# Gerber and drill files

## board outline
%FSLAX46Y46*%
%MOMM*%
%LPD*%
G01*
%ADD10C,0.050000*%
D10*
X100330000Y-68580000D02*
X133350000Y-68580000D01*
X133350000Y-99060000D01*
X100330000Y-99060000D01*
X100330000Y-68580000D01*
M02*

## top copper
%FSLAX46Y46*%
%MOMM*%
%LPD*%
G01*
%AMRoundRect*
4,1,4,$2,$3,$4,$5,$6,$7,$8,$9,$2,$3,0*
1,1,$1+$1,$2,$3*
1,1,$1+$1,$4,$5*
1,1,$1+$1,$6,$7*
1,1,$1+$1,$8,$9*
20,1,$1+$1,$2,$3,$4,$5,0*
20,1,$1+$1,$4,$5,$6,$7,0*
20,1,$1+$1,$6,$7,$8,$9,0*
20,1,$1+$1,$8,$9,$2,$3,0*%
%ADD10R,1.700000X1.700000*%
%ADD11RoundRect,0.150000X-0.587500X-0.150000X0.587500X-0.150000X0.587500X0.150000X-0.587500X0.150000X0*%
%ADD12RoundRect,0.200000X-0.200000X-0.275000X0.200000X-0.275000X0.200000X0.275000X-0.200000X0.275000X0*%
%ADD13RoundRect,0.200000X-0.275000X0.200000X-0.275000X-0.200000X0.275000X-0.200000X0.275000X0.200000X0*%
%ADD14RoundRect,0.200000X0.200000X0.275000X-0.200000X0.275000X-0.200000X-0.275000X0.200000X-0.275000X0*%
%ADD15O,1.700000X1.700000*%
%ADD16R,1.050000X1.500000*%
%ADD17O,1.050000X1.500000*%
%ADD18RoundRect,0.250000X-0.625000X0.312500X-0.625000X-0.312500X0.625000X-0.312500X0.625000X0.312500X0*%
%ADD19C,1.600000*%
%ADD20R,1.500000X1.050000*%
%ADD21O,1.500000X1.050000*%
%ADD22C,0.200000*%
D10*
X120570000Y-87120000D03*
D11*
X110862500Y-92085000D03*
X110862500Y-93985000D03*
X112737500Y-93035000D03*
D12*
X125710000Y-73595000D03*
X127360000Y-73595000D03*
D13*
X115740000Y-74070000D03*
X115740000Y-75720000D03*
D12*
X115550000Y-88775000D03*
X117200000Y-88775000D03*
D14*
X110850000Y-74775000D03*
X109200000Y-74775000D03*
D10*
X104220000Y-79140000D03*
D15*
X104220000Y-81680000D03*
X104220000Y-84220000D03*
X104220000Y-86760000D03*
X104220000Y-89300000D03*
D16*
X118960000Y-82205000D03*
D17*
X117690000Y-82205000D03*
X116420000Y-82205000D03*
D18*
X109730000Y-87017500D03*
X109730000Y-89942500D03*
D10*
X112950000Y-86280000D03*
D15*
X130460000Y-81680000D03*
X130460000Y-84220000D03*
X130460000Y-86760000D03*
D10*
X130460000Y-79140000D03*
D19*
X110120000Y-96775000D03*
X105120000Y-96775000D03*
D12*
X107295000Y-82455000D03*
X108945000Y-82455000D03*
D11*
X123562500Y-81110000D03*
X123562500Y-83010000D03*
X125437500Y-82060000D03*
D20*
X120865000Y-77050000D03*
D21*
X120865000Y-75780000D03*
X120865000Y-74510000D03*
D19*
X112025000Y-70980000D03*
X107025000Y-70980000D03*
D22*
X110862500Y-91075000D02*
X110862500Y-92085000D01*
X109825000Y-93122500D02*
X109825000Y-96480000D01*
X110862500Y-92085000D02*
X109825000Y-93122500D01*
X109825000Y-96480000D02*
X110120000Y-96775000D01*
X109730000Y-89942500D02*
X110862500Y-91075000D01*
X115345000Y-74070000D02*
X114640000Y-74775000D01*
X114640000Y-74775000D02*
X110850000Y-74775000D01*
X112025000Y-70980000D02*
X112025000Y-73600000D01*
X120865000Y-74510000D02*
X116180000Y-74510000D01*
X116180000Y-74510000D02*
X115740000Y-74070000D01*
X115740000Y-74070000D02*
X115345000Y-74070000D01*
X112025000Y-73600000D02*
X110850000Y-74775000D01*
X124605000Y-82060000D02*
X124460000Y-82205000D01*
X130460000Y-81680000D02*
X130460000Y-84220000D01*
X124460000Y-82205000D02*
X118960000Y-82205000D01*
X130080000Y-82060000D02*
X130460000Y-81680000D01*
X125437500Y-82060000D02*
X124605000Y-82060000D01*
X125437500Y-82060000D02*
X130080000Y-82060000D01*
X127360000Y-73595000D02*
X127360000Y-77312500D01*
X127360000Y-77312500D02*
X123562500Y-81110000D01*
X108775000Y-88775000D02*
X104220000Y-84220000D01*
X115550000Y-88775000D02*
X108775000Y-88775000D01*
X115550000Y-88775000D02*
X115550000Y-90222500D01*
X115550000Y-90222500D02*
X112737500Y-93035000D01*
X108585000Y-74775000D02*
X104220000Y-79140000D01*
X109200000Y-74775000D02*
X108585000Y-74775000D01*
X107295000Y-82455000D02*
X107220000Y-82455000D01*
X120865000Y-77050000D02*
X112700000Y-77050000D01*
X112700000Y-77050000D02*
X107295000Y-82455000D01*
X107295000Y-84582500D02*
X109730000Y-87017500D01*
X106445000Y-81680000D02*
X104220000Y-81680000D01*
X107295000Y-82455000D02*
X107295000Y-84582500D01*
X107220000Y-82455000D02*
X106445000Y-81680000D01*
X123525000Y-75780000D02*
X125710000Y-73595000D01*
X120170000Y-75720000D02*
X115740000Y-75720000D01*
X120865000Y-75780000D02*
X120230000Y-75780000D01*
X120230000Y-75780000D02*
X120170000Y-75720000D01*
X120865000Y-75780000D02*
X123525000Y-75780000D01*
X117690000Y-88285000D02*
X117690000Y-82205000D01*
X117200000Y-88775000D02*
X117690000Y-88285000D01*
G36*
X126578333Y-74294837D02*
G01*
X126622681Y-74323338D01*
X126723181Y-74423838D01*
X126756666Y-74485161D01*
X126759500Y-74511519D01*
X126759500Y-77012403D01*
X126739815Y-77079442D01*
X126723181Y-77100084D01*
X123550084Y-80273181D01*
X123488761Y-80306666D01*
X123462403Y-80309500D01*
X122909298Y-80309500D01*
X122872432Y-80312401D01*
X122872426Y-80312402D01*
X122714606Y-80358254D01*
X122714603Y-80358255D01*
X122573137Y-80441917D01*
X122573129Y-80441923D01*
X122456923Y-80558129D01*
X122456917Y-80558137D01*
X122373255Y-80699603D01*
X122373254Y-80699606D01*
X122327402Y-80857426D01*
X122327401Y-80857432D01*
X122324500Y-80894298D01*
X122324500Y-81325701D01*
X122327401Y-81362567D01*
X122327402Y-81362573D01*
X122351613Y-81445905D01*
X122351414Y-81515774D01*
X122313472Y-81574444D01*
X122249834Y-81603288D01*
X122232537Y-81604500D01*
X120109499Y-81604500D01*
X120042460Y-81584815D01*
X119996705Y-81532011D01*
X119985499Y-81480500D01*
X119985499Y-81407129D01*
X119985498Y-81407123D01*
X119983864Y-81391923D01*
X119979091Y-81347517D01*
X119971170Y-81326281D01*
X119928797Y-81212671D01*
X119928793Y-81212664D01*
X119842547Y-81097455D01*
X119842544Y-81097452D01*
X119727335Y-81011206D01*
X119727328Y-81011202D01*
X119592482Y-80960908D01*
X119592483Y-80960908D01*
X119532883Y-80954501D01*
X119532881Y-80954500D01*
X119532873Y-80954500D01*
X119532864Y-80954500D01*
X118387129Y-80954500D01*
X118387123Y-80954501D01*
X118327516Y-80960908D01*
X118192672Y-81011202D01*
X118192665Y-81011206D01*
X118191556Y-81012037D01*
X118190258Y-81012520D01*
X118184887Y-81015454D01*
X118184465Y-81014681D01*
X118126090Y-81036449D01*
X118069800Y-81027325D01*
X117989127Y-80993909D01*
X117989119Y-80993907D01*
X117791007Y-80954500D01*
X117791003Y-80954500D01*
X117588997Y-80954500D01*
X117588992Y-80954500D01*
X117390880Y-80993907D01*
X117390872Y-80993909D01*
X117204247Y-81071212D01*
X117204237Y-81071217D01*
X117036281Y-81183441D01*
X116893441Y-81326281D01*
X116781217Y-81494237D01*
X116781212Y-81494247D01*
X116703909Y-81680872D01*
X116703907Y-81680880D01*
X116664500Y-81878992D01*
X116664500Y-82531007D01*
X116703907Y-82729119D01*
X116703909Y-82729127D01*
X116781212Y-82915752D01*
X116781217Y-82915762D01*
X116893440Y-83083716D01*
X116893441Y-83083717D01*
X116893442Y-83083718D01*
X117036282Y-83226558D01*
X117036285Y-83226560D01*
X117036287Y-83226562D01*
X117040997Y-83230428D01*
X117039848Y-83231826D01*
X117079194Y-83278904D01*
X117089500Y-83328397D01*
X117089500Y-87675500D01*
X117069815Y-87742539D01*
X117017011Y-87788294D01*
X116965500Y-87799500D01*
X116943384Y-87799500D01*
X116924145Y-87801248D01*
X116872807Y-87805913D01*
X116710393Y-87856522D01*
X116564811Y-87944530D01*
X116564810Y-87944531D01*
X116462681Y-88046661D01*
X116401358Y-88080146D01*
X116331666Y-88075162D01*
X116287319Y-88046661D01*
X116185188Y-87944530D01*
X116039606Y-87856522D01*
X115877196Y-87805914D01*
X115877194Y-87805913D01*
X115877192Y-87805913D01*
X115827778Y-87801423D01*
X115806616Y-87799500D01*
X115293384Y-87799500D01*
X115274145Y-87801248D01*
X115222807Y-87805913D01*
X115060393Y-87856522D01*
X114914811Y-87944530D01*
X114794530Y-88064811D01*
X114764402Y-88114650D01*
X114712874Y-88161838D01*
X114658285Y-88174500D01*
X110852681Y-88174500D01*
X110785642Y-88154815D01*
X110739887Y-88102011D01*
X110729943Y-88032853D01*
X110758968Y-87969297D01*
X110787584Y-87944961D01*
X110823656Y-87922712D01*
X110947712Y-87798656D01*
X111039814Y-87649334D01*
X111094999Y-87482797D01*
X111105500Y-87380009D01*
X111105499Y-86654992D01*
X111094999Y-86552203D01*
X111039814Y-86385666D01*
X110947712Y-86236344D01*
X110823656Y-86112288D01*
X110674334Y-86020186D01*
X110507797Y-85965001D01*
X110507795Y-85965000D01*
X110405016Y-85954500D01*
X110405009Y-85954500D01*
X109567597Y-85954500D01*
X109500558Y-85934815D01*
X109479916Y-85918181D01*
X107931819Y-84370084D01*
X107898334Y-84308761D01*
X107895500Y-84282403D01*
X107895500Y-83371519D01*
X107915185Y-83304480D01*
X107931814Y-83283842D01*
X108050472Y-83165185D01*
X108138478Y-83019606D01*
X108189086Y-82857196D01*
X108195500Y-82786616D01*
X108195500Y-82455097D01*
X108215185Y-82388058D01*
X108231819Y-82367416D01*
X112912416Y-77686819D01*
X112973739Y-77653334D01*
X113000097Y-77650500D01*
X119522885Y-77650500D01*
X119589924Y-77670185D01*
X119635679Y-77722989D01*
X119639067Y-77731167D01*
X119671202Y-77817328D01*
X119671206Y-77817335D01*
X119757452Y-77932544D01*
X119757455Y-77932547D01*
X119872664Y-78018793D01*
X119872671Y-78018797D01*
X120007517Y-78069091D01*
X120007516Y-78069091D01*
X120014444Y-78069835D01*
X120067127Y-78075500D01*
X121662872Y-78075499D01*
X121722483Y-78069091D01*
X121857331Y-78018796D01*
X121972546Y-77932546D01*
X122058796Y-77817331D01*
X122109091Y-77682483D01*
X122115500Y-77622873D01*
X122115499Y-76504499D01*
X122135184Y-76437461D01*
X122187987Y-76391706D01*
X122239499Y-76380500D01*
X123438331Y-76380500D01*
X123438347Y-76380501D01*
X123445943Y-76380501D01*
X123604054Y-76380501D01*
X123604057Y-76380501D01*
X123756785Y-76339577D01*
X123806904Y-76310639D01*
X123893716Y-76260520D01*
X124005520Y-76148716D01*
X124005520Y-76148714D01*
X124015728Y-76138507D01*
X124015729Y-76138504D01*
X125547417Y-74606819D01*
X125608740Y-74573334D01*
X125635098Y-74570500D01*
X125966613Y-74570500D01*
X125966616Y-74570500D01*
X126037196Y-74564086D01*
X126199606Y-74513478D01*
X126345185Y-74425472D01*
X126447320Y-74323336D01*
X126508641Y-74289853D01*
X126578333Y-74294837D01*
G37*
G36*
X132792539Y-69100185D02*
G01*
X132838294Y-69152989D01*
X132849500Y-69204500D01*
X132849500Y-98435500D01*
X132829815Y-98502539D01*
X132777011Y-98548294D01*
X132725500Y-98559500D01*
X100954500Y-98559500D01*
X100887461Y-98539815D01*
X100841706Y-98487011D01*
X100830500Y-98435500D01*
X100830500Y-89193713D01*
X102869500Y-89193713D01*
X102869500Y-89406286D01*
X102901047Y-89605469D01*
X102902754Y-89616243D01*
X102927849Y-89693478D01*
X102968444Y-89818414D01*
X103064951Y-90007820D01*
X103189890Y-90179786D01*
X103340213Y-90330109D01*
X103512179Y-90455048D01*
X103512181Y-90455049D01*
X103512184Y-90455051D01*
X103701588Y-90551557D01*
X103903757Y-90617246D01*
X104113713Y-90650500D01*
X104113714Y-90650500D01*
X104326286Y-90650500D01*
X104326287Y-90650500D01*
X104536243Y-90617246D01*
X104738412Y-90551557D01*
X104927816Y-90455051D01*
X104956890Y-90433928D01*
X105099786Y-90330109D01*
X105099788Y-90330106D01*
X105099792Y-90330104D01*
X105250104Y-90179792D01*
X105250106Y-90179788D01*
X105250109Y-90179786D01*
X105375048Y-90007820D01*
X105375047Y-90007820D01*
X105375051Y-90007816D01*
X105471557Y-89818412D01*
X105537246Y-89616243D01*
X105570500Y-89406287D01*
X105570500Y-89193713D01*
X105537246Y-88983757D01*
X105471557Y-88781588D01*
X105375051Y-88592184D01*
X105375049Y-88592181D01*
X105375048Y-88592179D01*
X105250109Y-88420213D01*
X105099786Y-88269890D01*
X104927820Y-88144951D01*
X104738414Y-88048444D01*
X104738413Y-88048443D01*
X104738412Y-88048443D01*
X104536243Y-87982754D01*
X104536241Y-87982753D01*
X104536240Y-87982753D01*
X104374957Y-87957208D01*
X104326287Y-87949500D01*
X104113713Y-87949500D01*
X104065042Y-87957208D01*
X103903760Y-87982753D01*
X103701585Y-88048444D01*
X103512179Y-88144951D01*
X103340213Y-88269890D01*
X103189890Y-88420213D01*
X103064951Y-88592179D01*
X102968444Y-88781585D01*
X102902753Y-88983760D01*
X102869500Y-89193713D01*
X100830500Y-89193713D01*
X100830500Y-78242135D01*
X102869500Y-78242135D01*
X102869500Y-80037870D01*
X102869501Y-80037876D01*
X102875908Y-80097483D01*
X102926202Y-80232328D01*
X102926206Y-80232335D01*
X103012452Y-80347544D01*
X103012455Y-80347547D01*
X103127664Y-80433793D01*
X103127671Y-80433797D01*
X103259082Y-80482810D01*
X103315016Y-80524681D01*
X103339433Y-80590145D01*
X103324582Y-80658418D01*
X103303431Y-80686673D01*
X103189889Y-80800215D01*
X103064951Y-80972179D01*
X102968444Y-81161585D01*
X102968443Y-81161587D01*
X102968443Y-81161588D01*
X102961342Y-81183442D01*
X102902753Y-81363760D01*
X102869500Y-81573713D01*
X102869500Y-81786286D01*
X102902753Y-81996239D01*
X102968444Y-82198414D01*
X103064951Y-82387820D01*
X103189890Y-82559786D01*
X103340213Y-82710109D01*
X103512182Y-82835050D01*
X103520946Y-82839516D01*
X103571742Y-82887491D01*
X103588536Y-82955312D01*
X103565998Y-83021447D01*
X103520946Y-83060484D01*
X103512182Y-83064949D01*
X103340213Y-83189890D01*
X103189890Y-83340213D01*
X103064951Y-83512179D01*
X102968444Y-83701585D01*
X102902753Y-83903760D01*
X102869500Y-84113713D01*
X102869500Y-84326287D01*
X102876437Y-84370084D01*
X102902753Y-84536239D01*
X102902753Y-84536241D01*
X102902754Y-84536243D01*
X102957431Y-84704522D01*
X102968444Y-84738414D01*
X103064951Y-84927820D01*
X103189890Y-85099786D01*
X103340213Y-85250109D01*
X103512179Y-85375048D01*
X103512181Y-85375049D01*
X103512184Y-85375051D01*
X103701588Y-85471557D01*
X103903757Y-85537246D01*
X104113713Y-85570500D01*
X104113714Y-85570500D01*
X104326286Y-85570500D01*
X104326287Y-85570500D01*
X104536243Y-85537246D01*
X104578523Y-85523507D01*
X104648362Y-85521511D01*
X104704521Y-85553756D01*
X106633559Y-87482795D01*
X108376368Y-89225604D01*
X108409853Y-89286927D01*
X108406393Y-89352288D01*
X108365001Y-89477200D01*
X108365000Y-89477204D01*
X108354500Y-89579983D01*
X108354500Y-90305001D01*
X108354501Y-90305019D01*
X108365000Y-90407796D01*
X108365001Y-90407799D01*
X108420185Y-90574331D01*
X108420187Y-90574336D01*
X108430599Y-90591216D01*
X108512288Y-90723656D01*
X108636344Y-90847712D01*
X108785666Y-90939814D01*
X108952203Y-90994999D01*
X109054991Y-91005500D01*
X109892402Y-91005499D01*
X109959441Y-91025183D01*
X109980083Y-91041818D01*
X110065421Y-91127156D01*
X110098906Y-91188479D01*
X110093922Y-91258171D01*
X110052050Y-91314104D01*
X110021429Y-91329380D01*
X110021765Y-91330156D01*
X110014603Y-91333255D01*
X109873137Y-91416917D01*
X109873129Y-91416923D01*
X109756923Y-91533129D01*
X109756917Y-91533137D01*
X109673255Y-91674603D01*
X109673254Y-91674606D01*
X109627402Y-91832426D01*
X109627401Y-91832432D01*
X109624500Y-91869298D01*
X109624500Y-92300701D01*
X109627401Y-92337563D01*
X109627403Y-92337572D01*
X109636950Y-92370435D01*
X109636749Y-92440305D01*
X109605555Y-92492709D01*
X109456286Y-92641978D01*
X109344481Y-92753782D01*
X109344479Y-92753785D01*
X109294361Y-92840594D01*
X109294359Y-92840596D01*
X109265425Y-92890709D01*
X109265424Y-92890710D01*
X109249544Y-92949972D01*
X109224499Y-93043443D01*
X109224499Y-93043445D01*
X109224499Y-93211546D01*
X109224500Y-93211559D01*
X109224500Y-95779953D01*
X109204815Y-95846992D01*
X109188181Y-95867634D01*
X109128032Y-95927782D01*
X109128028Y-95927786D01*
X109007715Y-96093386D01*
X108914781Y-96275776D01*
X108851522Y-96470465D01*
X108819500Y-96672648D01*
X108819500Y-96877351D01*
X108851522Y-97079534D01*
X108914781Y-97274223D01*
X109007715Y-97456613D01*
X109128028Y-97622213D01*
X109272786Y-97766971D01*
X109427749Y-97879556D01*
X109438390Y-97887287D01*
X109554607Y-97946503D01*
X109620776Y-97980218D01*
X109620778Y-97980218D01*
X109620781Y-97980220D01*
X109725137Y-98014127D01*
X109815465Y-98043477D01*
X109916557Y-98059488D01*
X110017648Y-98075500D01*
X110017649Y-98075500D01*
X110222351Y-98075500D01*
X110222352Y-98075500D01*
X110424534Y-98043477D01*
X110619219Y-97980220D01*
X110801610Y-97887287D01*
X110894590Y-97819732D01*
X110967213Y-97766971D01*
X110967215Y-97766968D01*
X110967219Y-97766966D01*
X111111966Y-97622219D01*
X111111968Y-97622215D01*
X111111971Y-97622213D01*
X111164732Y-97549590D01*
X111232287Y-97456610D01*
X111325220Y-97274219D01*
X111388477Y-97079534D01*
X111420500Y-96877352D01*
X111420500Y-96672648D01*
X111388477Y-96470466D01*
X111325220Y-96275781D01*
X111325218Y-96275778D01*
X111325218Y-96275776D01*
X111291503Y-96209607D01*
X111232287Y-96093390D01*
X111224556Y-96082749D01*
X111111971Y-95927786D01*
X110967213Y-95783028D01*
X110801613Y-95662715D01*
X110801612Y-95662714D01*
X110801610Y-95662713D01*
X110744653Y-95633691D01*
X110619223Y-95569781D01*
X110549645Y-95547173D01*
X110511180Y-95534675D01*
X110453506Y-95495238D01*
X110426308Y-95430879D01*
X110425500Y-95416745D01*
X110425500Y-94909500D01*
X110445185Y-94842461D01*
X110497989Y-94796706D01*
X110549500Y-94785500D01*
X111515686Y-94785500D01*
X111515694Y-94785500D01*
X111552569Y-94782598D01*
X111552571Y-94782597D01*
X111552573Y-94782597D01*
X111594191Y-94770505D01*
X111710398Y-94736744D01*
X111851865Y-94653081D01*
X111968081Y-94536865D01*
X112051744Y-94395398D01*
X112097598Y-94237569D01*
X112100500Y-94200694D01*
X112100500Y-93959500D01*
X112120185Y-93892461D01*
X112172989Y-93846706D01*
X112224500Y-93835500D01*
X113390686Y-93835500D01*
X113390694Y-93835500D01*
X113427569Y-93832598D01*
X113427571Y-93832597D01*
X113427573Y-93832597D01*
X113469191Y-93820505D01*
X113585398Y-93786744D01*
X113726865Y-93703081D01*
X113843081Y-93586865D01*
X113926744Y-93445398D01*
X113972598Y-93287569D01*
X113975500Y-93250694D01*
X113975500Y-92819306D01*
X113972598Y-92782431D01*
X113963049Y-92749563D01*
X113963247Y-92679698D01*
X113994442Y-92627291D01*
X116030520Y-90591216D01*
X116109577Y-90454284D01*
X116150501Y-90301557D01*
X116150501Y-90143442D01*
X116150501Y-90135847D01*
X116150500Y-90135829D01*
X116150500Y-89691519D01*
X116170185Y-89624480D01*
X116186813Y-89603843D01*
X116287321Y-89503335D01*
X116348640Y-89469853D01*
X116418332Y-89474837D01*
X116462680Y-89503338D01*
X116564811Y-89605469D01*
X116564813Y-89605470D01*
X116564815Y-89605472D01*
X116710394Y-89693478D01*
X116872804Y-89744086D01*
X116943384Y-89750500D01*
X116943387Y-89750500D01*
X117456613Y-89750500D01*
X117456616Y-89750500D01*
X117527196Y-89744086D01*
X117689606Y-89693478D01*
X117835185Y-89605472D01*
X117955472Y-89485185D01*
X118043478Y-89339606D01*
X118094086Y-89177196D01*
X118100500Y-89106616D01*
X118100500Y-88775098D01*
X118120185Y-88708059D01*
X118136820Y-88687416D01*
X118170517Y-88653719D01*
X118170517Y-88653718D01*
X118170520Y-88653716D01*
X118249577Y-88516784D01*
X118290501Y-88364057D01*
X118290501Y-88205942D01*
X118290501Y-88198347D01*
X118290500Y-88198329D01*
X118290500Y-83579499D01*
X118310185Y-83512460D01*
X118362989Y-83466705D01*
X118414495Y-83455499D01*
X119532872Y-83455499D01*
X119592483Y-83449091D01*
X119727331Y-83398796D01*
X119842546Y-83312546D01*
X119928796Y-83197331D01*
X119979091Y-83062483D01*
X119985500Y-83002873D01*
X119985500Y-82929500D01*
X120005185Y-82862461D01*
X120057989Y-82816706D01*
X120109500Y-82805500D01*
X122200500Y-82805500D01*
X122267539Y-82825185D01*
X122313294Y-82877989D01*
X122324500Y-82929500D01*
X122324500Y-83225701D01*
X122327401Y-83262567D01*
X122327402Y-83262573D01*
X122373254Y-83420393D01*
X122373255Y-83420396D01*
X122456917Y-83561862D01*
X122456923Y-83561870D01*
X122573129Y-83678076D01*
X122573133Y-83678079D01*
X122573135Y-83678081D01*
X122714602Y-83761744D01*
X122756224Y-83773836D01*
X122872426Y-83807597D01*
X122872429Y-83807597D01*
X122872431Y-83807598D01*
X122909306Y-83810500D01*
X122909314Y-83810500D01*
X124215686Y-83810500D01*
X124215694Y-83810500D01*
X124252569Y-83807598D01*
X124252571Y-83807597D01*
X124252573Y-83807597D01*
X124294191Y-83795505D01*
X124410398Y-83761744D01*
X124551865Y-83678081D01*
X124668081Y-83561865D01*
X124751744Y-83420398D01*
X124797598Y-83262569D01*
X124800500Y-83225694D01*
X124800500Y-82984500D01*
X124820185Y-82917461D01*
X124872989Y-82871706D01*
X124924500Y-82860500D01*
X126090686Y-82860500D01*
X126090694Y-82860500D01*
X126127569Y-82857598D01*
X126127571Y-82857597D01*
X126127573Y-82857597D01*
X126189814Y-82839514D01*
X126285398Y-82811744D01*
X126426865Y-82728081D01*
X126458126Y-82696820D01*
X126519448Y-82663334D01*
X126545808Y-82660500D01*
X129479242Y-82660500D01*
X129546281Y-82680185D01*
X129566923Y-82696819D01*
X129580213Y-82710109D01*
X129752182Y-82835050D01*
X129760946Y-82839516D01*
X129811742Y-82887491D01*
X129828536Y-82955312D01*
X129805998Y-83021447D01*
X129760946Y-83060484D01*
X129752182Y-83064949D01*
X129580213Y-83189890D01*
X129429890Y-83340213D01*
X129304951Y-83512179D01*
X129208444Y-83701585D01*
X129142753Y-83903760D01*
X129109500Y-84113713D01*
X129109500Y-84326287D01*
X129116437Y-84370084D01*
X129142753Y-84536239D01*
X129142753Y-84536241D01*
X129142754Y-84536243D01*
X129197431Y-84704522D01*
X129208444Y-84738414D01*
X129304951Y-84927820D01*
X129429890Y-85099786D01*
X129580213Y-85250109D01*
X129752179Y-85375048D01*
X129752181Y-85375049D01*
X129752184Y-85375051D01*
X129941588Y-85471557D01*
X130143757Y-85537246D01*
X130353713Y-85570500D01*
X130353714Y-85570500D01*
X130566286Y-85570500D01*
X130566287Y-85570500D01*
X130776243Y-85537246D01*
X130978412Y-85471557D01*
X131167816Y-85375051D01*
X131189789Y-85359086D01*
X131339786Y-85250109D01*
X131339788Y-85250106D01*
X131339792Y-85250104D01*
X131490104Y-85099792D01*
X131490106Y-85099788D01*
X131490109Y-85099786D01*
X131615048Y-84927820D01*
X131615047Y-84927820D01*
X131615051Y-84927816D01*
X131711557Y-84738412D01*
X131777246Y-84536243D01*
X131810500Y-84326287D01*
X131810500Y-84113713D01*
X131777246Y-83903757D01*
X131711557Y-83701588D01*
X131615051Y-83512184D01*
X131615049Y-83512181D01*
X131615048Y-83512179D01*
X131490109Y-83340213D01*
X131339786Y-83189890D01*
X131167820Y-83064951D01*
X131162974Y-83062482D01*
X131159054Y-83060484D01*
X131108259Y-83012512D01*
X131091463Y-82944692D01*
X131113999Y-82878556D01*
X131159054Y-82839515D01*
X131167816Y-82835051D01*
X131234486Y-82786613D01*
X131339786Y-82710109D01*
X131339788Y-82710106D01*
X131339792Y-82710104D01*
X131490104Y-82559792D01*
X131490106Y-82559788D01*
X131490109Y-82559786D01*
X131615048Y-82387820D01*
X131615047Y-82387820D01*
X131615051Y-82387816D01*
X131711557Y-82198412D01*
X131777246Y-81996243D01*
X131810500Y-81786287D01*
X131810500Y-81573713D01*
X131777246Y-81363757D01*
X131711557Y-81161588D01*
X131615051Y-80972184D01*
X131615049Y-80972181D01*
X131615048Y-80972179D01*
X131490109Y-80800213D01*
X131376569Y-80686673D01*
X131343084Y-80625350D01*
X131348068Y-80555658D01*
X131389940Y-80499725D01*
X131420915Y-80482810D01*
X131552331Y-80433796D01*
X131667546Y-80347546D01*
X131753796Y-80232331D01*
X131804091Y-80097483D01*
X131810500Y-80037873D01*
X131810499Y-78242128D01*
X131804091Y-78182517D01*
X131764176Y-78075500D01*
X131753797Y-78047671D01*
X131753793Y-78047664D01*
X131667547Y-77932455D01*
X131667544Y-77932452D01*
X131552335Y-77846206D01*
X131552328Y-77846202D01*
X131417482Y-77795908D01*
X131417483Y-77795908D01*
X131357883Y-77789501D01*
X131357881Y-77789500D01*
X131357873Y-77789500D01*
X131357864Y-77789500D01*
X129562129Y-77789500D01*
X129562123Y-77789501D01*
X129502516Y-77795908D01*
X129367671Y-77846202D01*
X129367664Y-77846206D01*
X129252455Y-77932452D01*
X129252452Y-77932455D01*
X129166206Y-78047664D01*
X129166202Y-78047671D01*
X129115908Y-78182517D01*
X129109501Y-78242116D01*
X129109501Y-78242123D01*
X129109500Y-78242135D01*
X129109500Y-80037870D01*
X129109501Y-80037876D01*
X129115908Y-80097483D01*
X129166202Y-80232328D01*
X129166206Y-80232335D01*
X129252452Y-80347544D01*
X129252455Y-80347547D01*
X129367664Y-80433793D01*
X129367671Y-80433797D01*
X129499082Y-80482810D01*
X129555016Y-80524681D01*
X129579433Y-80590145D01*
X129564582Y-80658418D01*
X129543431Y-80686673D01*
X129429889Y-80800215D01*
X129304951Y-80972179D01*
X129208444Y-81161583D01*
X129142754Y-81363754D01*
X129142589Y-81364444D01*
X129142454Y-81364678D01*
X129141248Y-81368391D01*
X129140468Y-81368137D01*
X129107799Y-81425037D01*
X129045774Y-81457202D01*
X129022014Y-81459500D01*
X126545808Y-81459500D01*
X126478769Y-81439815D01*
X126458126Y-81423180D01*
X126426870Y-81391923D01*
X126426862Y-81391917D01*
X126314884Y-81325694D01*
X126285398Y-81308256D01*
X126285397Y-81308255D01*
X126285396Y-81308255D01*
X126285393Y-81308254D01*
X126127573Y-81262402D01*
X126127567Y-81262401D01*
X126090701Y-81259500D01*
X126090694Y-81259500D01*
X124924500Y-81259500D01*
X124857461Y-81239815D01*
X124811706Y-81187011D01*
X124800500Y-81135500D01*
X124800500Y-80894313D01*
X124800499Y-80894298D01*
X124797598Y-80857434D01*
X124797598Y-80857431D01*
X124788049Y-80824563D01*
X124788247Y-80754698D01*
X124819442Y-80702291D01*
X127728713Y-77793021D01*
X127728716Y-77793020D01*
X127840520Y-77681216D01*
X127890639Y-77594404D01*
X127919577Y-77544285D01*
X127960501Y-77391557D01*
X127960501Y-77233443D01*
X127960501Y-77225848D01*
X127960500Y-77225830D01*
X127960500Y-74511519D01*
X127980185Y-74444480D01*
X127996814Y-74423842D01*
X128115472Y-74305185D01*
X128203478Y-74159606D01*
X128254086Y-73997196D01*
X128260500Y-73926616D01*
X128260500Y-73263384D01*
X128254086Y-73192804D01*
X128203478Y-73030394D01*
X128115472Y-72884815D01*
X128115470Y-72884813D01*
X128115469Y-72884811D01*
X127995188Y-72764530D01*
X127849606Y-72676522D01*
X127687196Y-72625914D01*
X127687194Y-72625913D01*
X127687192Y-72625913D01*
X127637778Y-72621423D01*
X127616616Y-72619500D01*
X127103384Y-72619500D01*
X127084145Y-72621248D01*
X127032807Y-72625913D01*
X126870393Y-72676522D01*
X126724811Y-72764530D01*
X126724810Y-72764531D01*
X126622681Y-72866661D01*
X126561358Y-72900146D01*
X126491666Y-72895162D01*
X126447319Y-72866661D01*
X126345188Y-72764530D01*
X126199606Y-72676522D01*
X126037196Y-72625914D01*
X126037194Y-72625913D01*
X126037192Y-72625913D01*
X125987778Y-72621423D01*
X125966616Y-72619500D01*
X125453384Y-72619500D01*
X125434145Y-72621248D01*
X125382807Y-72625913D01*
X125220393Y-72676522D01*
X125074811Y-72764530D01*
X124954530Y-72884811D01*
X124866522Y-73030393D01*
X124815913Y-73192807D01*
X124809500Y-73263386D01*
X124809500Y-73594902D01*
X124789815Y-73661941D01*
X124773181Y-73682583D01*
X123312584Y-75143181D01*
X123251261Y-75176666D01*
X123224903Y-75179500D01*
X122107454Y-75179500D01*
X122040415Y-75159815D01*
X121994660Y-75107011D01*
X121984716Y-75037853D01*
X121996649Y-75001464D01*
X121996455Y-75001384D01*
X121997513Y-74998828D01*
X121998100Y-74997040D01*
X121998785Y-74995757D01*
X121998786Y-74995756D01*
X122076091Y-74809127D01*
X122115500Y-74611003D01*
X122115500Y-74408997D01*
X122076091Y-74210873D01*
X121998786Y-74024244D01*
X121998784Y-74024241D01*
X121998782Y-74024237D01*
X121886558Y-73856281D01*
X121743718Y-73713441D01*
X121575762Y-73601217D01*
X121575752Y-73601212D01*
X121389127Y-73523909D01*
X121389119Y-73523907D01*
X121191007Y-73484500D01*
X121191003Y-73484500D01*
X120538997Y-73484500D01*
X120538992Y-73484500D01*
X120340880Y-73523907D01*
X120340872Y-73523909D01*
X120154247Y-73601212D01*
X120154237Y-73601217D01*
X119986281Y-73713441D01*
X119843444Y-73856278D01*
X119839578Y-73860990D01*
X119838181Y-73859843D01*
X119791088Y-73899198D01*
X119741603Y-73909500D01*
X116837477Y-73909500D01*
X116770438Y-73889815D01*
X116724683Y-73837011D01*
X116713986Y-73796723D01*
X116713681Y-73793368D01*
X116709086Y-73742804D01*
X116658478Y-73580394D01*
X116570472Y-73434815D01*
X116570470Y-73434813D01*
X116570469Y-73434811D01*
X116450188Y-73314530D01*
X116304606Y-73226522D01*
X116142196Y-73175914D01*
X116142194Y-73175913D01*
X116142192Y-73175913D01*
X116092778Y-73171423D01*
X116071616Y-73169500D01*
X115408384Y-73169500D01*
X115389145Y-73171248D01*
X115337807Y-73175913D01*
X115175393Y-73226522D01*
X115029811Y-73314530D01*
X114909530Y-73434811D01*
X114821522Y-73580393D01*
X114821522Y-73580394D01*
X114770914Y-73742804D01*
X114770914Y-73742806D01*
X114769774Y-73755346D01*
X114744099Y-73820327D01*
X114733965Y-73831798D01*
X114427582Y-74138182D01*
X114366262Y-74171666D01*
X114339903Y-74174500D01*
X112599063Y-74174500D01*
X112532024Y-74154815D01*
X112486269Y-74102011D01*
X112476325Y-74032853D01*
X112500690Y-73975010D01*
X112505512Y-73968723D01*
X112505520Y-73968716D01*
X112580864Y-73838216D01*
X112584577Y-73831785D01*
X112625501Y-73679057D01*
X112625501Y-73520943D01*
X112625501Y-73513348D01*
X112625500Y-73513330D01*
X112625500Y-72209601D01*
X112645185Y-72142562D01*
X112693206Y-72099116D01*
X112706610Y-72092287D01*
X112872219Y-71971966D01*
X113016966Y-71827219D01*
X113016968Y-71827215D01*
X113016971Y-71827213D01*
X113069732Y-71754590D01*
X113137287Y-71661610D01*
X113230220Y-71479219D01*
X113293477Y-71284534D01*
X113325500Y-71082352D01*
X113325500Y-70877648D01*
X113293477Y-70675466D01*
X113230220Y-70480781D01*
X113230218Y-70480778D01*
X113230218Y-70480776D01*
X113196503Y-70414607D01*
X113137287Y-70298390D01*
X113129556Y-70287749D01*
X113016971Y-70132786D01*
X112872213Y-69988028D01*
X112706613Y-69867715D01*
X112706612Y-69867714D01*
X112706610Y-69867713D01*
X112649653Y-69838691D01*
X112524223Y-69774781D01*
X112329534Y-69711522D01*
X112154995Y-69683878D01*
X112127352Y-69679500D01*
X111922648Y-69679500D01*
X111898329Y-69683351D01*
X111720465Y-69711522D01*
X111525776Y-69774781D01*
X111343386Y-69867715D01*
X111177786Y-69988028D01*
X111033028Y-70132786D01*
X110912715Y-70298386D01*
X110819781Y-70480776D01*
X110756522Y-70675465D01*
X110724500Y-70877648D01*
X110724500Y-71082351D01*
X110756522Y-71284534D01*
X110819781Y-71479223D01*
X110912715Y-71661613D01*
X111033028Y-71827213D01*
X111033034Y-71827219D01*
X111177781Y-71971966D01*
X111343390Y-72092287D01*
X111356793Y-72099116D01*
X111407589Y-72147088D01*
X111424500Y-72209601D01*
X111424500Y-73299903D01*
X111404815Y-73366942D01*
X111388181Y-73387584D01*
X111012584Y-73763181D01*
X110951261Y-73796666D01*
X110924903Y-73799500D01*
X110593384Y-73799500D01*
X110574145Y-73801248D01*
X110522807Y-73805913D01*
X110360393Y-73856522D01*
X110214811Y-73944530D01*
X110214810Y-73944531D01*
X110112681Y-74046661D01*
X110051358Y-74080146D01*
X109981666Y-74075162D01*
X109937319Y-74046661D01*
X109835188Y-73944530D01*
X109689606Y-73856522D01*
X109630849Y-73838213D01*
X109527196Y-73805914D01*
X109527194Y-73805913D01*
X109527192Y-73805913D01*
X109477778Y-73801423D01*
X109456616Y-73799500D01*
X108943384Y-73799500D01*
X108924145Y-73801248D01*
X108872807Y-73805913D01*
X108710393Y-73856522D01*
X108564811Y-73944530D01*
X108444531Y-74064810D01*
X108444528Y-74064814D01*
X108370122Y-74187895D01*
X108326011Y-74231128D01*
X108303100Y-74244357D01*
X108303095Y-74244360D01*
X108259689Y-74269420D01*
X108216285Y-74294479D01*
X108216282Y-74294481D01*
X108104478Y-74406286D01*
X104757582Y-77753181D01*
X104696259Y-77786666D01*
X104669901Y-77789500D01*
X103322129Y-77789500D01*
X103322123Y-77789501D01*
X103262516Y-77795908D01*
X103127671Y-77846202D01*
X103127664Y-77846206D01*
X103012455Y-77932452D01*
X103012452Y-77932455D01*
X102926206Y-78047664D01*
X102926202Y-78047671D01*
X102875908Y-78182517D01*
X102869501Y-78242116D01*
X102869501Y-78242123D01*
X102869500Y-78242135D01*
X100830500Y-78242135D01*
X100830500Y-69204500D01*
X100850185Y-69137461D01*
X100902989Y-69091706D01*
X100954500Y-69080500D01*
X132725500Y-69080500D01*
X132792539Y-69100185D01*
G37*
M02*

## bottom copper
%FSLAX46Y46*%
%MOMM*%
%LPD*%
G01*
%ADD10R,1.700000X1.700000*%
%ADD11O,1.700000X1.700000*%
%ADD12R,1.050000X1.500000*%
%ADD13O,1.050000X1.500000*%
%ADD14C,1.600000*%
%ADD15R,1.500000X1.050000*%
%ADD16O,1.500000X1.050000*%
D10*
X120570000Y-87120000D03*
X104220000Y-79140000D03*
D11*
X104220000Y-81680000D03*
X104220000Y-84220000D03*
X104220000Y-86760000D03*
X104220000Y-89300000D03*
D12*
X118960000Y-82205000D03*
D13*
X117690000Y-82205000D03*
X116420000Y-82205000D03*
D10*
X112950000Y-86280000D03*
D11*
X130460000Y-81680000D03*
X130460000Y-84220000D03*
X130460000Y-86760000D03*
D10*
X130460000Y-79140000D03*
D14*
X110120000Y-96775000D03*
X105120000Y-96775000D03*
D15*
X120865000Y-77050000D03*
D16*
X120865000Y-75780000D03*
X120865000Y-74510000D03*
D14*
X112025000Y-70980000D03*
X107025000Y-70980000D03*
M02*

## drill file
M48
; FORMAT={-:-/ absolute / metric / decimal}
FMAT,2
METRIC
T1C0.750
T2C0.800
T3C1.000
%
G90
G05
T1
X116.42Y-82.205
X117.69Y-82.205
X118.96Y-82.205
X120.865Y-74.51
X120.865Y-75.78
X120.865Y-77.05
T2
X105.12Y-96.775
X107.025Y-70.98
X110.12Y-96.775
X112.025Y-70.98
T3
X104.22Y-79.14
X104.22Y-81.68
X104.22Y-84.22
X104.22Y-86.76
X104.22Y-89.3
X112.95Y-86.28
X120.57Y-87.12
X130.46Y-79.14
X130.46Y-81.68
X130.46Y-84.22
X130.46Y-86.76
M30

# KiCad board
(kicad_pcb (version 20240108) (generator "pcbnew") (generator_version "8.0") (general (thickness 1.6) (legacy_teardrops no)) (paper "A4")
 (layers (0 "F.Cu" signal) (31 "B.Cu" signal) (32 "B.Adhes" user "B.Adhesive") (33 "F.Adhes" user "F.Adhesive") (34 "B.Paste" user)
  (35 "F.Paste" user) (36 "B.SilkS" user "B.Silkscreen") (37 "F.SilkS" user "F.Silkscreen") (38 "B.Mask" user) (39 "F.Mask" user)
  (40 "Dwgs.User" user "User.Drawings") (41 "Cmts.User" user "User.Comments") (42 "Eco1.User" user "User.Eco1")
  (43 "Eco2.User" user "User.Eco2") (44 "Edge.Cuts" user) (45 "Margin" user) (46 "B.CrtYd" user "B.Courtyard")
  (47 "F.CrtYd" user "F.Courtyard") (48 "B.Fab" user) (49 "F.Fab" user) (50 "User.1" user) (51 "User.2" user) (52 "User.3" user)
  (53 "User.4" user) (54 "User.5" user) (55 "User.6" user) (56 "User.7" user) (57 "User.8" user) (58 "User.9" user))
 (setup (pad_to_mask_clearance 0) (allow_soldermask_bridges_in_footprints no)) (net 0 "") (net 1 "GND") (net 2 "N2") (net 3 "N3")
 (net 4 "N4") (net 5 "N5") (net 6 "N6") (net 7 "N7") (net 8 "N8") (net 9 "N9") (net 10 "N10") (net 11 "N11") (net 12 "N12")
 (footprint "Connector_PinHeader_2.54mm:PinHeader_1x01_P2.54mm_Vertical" (layer "F.Cu") (at 120.57 87.12)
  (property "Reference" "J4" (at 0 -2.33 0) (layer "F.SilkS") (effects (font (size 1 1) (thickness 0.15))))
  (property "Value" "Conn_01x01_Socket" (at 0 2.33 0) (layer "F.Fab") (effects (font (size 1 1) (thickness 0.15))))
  (pad "1" thru_hole rect (at 0 0) (size 1.7 1.7) (drill 1) (layers "*.Cu" "*.Mask") (remove_unused_layers no) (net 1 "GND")))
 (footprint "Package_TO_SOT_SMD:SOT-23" (layer "F.Cu") (at 111.8 93.035)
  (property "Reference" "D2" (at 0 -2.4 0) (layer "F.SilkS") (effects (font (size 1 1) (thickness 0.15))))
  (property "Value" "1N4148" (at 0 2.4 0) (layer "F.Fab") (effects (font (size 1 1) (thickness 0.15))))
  (pad "1" smd roundrect (at -0.9375 -0.95) (size 1.475 0.6) (layers "F.Cu" "F.Paste" "F.Mask") (roundrect_rratio 0.25) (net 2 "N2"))
  (pad "2" smd roundrect (at -0.9375 0.95) (size 1.475 0.6) (layers "F.Cu" "F.Paste" "F.Mask") (roundrect_rratio 0.25))
  (pad "3" smd roundrect (at 0.9375 0) (size 1.475 0.6) (layers "F.Cu" "F.Paste" "F.Mask") (roundrect_rratio 0.25) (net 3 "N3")))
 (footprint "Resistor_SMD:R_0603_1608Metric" (layer "F.Cu") (at 126.535 73.595)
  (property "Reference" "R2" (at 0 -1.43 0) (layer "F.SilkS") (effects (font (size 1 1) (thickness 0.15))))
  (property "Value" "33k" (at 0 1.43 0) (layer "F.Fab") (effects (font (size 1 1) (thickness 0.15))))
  (pad "1" smd roundrect (at -0.825 0) (size 0.8 0.95) (layers "F.Cu" "F.Paste" "F.Mask") (roundrect_rratio 0.25) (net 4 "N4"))
  (pad "2" smd roundrect (at 0.825 0) (size 0.8 0.95) (layers "F.Cu" "F.Paste" "F.Mask") (roundrect_rratio 0.25) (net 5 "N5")))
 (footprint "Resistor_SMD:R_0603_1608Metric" (layer "F.Cu") (at 115.74 74.895 -90)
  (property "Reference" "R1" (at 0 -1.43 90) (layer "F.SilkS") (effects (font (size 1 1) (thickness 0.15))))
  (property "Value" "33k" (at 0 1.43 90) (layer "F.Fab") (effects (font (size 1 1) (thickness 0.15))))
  (pad "1" smd roundrect (at -0.825 0 270) (size 0.8 0.95) (layers "F.Cu" "F.Paste" "F.Mask") (roundrect_rratio 0.25) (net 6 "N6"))
  (pad "2" smd roundrect (at 0.825 0 270) (size 0.8 0.95) (layers "F.Cu" "F.Paste" "F.Mask") (roundrect_rratio 0.25) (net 4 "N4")))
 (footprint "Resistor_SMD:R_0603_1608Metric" (layer "F.Cu") (at 116.375 88.775)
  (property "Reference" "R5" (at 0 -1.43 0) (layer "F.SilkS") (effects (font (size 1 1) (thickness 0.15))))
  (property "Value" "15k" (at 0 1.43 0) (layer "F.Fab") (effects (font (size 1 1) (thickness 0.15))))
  (pad "1" smd roundrect (at -0.825 0) (size 0.8 0.95) (layers "F.Cu" "F.Paste" "F.Mask") (roundrect_rratio 0.25) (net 3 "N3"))
  (pad "2" smd roundrect (at 0.825 0) (size 0.8 0.95) (layers "F.Cu" "F.Paste" "F.Mask") (roundrect_rratio 0.25) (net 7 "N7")))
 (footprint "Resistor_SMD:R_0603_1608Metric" (layer "F.Cu") (at 110.025 74.775 180)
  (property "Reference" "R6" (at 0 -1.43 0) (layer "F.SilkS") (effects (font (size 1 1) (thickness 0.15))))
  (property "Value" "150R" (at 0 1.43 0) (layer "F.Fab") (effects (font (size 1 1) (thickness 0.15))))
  (pad "1" smd roundrect (at -0.825 0 180) (size 0.8 0.95) (layers "F.Cu" "F.Paste" "F.Mask") (roundrect_rratio 0.25) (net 6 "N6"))
  (pad "2" smd roundrect (at 0.825 0 180) (size 0.8 0.95) (layers "F.Cu" "F.Paste" "F.Mask") (roundrect_rratio 0.25) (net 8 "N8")))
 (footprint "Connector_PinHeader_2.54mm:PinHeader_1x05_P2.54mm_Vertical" (layer "F.Cu") (at 104.22 79.14)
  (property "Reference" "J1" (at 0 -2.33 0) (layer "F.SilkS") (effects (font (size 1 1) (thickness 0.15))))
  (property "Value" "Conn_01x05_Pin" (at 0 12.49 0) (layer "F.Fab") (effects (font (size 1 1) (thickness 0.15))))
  (pad "1" thru_hole rect (at 0 0) (size 1.7 1.7) (drill 1) (layers "*.Cu" "*.Mask") (remove_unused_layers no) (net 8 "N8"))
  (pad "2" thru_hole oval (at 0 2.54) (size 1.7 1.7) (drill 1) (layers "*.Cu" "*.Mask") (remove_unused_layers no) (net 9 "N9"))
  (pad "3" thru_hole oval (at 0 5.08) (size 1.7 1.7) (drill 1) (layers "*.Cu" "*.Mask") (remove_unused_layers no) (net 3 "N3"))
  (pad "4" thru_hole oval (at 0 7.62) (size 1.7 1.7) (drill 1) (layers "*.Cu" "*.Mask") (remove_unused_layers no) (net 1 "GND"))
  (pad "5" thru_hole oval (at 0 10.16) (size 1.7 1.7) (drill 1) (layers "*.Cu" "*.Mask") (remove_unused_layers no) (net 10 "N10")))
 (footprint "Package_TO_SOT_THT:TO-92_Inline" (layer "F.Cu") (at 118.96 82.205 180)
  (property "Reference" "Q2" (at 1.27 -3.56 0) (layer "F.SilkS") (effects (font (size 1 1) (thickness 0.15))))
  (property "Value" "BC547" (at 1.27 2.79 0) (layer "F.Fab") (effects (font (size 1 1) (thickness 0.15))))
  (pad "1" thru_hole rect (at 0 0 180) (size 1.05 1.5) (drill 0.75) (layers "*.Cu" "*.Mask") (remove_unused_layers no) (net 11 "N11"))
  (pad "2" thru_hole oval (at 1.27 0 180) (size 1.05 1.5) (drill 0.75) (layers "*.Cu" "*.Mask") (remove_unused_layers no) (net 7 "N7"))
  (pad "3" thru_hole oval (at 2.54 0 180) (size 1.05 1.5) (drill 0.75) (layers "*.Cu" "*.Mask") (remove_unused_layers no) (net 1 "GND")))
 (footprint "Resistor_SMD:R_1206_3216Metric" (layer "F.Cu") (at 109.73 88.48 -90)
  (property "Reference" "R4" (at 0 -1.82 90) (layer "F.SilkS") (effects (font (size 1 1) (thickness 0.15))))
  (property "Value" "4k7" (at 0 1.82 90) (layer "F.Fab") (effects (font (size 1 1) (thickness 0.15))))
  (pad "1" smd roundrect (at -1.4625 0 270) (size 1.125 1.75) (layers "F.Cu" "F.Paste" "F.Mask") (roundrect_rratio 0.222222) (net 9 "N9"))
  (pad "2" smd roundrect (at 1.4625 0 270) (size 1.125 1.75) (layers "F.Cu" "F.Paste" "F.Mask") (roundrect_rratio 0.222222) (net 2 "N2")))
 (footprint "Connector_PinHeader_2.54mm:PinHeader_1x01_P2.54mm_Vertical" (layer "F.Cu") (at 112.95 86.28)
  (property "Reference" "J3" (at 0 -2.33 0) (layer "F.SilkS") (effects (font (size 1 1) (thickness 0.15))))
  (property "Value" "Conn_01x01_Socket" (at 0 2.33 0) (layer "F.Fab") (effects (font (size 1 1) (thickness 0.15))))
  (pad "1" thru_hole rect (at 0 0) (size 1.7 1.7) (drill 1) (layers "*.Cu" "*.Mask") (remove_unused_layers no) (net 1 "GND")))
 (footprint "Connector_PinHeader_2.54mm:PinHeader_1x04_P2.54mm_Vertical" (layer "F.Cu") (at 130.46 79.14)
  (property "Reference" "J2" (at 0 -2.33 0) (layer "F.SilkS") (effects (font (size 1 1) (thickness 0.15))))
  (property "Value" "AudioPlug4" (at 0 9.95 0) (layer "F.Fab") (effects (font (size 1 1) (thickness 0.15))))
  (pad "R1" thru_hole oval (at 0 2.54) (size 1.7 1.7) (drill 1) (layers "*.Cu" "*.Mask") (remove_unused_layers no) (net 11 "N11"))
  (pad "R2" thru_hole oval (at 0 5.08) (size 1.7 1.7) (drill 1) (layers "*.Cu" "*.Mask") (remove_unused_layers no) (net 11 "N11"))
  (pad "S" thru_hole oval (at 0 7.62) (size 1.7 1.7) (drill 1) (layers "*.Cu" "*.Mask") (remove_unused_layers no) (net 1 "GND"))
  (pad "T" thru_hole rect (at 0 0) (size 1.7 1.7) (drill 1) (layers "*.Cu" "*.Mask") (remove_unused_layers no) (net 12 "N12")))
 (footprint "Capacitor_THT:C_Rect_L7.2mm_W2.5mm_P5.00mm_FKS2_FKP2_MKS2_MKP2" (layer "F.Cu") (at 110.12 96.775 180)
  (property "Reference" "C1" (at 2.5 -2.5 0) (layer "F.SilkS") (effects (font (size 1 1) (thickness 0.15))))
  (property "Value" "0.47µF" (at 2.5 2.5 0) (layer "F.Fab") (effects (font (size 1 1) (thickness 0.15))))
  (pad "1" thru_hole circle (at 0 0 180) (size 1.6 1.6) (drill 0.8) (layers "*.Cu" "*.Mask") (remove_unused_layers no) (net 2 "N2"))
  (pad "2" thru_hole circle (at 5 0 180) (size 1.6 1.6) (drill 0.8) (layers "*.Cu" "*.Mask") (remove_unused_layers no) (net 1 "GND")))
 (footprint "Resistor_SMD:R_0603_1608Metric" (layer "F.Cu") (at 108.12 82.455)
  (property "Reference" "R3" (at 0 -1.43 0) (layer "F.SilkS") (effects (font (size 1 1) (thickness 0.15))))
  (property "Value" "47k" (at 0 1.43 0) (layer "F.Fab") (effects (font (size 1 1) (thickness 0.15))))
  (pad "1" smd roundrect (at -0.825 0) (size 0.8 0.95) (layers "F.Cu" "F.Paste" "F.Mask") (roundrect_rratio 0.25) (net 9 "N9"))
  (pad "2" smd roundrect (at 0.825 0) (size 0.8 0.95) (layers "F.Cu" "F.Paste" "F.Mask") (roundrect_rratio 0.25) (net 1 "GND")))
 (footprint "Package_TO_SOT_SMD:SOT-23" (layer "F.Cu") (at 124.5 82.06)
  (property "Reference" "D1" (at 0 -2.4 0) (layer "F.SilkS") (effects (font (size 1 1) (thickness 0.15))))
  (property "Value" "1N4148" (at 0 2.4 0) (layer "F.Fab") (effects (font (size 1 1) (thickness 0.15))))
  (pad "1" smd roundrect (at -0.9375 -0.95) (size 1.475 0.6) (layers "F.Cu" "F.Paste" "F.Mask") (roundrect_rratio 0.25) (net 5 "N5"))
  (pad "2" smd roundrect (at -0.9375 0.95) (size 1.475 0.6) (layers "F.Cu" "F.Paste" "F.Mask") (roundrect_rratio 0.25))
  (pad "3" smd roundrect (at 0.9375 0) (size 1.475 0.6) (layers "F.Cu" "F.Paste" "F.Mask") (roundrect_rratio 0.25) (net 11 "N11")))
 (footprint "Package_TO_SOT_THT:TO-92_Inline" (layer "F.Cu") (at 120.865 77.05 90)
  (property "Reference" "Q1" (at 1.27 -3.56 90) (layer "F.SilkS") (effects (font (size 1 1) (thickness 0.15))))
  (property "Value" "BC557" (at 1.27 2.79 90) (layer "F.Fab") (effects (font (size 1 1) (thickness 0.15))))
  (pad "1" thru_hole rect (at 0 0 90) (size 1.05 1.5) (drill 0.75) (layers "*.Cu" "*.Mask") (remove_unused_layers no) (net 9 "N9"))
  (pad "2" thru_hole oval (at 1.27 0 90) (size 1.05 1.5) (drill 0.75) (layers "*.Cu" "*.Mask") (remove_unused_layers no) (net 4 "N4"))
  (pad "3" thru_hole oval (at 2.54 0 90) (size 1.05 1.5) (drill 0.75) (layers "*.Cu" "*.Mask") (remove_unused_layers no) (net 6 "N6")))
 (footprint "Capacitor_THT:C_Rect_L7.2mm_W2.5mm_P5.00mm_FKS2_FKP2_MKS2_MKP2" (layer "F.Cu") (at 112.025 70.98 180)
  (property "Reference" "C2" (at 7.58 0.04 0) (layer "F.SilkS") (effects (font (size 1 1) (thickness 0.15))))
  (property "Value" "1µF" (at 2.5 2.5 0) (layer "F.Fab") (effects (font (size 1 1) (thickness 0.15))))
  (pad "1" thru_hole circle (at 0 0 180) (size 1.6 1.6) (drill 0.8) (layers "*.Cu" "*.Mask") (remove_unused_layers no) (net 6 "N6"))
  (pad "2" thru_hole circle (at 5 0 180) (size 1.6 1.6) (drill 0.8) (layers "*.Cu" "*.Mask") (remove_unused_layers no) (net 1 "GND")))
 (gr_rect (start 100.33 68.58) (end 133.35 99.06) (stroke (width 0.05) (type default)) (fill none) (layer "Edge.Cuts"))
 (segment (start 110.8625 91.075) (end 110.8625 92.085) (width 0.2) (layer "F.Cu") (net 2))
 (segment (start 109.825 93.1225) (end 109.825 96.48) (width 0.2) (layer "F.Cu") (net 2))
 (segment (start 110.8625 92.085) (end 109.825 93.1225) (width 0.2) (layer "F.Cu") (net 2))
 (segment (start 109.825 96.48) (end 110.12 96.775) (width 0.2) (layer "F.Cu") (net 2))
 (segment (start 109.73 89.9425) (end 110.8625 91.075) (width 0.2) (layer "F.Cu") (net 2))
 (segment (start 115.345 74.07) (end 114.64 74.775) (width 0.2) (layer "F.Cu") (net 6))
 (segment (start 114.64 74.775) (end 110.85 74.775) (width 0.2) (layer "F.Cu") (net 6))
 (segment (start 112.025 70.98) (end 112.025 73.6) (width 0.2) (layer "F.Cu") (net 6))
 (segment (start 120.865 74.51) (end 116.18 74.51) (width 0.2) (layer "F.Cu") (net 6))
 (segment (start 116.18 74.51) (end 115.74 74.07) (width 0.2) (layer "F.Cu") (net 6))
 (segment (start 115.74 74.07) (end 115.345 74.07) (width 0.2) (layer "F.Cu") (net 6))
 (segment (start 112.025 73.6) (end 110.85 74.775) (width 0.2) (layer "F.Cu") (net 6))
 (segment (start 124.605 82.06) (end 124.46 82.205) (width 0.2) (layer "F.Cu") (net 11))
 (segment (start 130.46 81.68) (end 130.46 84.22) (width 0.2) (layer "F.Cu") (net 11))
 (segment (start 124.46 82.205) (end 118.96 82.205) (width 0.2) (layer "F.Cu") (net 11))
 (segment (start 130.08 82.06) (end 130.46 81.68) (width 0.2) (layer "F.Cu") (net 11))
 (segment (start 125.4375 82.06) (end 124.605 82.06) (width 0.2) (layer "F.Cu") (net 11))
 (segment (start 125.4375 82.06) (end 130.08 82.06) (width 0.2) (layer "F.Cu") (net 11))
 (segment (start 127.36 73.595) (end 127.36 77.3125) (width 0.2) (layer "F.Cu") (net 5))
 (segment (start 127.36 77.3125) (end 123.5625 81.11) (width 0.2) (layer "F.Cu") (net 5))
 (segment (start 108.775 88.775) (end 104.22 84.22) (width 0.2) (layer "F.Cu") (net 3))
 (segment (start 115.55 88.775) (end 108.775 88.775) (width 0.2) (layer "F.Cu") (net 3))
 (segment (start 115.55 88.775) (end 115.55 90.2225) (width 0.2) (layer "F.Cu") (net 3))
 (segment (start 115.55 90.2225) (end 112.7375 93.035) (width 0.2) (layer "F.Cu") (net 3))
 (segment (start 108.585 74.775) (end 104.22 79.14) (width 0.2) (layer "F.Cu") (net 8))
 (segment (start 109.2 74.775) (end 108.585 74.775) (width 0.2) (layer "F.Cu") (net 8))
 (segment (start 107.295 82.455) (end 107.22 82.455) (width 0.2) (layer "F.Cu") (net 9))
 (segment (start 120.865 77.05) (end 112.7 77.05) (width 0.2) (layer "F.Cu") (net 9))
 (segment (start 112.7 77.05) (end 107.295 82.455) (width 0.2) (layer "F.Cu") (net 9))
 (segment (start 107.295 84.5825) (end 109.73 87.0175) (width 0.2) (layer "F.Cu") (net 9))
 (segment (start 106.445 81.68) (end 104.22 81.68) (width 0.2) (layer "F.Cu") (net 9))
 (segment (start 107.295 82.455) (end 107.295 84.5825) (width 0.2) (layer "F.Cu") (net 9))
 (segment (start 107.22 82.455) (end 106.445 81.68) (width 0.2) (layer "F.Cu") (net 9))
 (segment (start 123.525 75.78) (end 125.71 73.595) (width 0.2) (layer "F.Cu") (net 4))
 (segment (start 120.17 75.72) (end 115.74 75.72) (width 0.2) (layer "F.Cu") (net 4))
 (segment (start 120.865 75.78) (end 120.23 75.78) (width 0.2) (layer "F.Cu") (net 4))
 (segment (start 120.23 75.78) (end 120.17 75.72) (width 0.2) (layer "F.Cu") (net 4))
 (segment (start 120.865 75.78) (end 123.525 75.78) (width 0.2) (layer "F.Cu") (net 4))
 (segment (start 117.69 88.285) (end 117.69 82.205) (width 0.2) (layer "F.Cu") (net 7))
 (segment (start 117.2 88.775) (end 117.69 88.285) (width 0.2) (layer "F.Cu") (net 7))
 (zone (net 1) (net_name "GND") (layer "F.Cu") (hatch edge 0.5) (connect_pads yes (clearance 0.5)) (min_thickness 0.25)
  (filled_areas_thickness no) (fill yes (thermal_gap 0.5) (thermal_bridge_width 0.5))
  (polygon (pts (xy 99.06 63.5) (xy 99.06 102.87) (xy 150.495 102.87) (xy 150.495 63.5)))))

